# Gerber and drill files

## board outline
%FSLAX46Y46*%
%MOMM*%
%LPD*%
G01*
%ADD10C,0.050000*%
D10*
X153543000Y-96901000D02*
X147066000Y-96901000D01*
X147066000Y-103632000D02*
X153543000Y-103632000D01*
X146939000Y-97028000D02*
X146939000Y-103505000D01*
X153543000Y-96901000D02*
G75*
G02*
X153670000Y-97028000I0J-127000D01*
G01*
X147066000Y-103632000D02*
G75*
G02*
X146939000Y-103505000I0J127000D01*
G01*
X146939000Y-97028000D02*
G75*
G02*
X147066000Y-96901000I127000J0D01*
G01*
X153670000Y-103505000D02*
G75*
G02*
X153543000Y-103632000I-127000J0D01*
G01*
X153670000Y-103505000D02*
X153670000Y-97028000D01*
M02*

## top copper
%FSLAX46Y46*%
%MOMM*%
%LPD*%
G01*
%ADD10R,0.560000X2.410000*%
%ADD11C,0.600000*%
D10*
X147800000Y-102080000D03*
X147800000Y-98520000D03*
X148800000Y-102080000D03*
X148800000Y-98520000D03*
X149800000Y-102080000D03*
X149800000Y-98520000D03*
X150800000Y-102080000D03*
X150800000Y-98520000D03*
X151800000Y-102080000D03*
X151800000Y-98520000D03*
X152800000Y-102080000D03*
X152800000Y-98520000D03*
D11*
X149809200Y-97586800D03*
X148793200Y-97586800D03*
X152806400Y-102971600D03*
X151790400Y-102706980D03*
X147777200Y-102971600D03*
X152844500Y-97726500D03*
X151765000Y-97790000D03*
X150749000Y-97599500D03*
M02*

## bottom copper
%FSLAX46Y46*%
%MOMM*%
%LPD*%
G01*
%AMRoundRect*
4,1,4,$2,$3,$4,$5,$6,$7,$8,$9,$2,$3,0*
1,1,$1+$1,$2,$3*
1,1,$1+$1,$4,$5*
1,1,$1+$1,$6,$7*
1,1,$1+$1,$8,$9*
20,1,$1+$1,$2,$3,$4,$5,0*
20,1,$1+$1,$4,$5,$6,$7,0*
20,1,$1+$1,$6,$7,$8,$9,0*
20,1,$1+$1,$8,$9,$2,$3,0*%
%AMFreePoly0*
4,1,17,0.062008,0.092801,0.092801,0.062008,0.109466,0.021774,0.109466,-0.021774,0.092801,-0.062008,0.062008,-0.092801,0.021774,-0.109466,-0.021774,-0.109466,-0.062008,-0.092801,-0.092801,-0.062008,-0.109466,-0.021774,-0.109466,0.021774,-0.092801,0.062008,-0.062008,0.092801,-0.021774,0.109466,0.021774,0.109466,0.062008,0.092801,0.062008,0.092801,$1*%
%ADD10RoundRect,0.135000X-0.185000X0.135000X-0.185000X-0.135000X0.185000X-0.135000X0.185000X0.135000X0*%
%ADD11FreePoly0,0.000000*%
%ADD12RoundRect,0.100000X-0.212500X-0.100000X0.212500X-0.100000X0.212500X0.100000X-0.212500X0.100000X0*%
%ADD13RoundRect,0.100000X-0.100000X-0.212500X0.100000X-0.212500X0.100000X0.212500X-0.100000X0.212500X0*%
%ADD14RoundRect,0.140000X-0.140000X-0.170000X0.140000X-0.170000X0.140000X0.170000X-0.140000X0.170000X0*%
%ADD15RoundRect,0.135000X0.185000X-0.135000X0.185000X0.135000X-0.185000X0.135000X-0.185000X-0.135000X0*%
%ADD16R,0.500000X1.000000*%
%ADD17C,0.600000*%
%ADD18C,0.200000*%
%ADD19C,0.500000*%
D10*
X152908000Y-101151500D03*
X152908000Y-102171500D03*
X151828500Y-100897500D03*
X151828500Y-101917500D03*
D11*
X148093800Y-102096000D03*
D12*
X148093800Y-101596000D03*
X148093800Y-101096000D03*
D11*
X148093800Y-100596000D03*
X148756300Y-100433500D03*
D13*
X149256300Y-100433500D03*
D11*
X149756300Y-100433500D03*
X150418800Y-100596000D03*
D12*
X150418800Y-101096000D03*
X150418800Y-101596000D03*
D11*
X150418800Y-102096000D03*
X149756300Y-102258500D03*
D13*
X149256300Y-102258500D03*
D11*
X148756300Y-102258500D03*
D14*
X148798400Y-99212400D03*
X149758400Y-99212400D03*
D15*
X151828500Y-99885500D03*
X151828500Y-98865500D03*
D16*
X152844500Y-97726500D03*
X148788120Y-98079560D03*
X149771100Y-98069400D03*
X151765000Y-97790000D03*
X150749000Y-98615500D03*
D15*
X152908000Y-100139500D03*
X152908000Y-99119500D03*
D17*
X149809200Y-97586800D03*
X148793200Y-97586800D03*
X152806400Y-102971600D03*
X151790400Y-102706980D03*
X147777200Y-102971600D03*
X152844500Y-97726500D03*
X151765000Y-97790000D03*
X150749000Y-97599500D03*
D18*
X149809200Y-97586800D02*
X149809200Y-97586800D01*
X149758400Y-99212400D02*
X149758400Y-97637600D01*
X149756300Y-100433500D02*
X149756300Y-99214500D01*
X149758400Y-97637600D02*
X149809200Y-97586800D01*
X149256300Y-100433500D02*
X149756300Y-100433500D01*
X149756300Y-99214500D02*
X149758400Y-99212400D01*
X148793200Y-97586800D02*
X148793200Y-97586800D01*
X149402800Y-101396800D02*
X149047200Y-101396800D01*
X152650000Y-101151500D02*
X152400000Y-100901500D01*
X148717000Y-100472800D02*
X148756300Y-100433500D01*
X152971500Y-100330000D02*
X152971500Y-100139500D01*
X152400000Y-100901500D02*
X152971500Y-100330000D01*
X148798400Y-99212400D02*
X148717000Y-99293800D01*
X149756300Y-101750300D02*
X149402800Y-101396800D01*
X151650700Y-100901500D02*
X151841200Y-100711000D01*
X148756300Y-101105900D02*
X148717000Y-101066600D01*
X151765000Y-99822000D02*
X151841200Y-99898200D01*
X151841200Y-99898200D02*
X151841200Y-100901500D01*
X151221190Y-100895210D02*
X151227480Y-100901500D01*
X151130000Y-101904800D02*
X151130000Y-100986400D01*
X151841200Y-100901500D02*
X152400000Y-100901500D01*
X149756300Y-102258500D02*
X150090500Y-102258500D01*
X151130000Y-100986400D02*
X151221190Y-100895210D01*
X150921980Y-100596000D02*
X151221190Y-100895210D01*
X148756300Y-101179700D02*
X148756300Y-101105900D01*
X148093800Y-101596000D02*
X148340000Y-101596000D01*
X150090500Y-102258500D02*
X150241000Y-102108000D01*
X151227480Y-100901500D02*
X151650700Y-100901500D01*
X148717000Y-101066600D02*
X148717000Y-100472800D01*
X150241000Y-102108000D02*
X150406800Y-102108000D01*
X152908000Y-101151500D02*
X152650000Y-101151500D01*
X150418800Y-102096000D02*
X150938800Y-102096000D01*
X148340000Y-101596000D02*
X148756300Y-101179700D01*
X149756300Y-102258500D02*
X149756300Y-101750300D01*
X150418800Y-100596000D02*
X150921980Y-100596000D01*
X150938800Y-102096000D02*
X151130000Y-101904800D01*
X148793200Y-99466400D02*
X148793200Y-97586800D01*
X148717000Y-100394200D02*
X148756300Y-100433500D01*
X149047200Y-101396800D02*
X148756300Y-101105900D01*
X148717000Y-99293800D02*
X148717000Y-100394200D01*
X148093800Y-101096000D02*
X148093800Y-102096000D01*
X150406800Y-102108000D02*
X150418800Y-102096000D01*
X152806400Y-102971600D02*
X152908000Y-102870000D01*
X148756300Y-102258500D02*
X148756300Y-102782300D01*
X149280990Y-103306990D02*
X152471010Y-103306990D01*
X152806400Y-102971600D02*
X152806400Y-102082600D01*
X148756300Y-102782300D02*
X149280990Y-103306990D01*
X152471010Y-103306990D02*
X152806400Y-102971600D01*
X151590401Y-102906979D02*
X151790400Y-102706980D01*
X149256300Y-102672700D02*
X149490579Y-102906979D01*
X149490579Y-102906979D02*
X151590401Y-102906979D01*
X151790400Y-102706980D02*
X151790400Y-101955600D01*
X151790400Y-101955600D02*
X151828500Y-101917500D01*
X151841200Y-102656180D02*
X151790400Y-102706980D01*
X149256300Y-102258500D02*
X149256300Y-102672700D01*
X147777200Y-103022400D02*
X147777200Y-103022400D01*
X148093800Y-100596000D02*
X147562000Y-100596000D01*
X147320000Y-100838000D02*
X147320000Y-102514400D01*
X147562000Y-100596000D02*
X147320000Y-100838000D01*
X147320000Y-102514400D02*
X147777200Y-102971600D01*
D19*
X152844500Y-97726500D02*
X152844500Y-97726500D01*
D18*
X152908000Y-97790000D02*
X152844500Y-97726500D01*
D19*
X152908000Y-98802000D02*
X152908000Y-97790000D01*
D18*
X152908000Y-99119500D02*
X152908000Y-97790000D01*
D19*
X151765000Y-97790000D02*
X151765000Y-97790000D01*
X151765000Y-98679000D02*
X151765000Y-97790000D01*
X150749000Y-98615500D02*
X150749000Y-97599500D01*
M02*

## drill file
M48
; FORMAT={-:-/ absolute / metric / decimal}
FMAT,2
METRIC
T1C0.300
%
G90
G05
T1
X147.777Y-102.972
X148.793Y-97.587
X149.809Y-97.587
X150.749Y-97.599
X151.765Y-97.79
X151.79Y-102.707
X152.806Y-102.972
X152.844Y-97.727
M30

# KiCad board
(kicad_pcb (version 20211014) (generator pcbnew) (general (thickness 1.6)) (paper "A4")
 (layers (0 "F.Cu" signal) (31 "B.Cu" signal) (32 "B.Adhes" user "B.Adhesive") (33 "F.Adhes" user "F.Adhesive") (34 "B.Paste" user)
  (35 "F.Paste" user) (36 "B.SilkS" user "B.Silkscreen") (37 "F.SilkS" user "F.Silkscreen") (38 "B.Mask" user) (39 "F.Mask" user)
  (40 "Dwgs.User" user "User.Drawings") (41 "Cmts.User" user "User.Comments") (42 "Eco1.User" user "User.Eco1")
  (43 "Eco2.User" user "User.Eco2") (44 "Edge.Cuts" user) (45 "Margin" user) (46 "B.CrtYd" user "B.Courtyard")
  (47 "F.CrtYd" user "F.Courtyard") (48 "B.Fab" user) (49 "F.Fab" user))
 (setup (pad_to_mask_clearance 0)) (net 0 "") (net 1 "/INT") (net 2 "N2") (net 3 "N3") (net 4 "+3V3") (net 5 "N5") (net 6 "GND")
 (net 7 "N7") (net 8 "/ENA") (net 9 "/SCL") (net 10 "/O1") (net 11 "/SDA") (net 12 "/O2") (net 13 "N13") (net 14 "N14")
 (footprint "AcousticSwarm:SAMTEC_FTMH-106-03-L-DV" (layer "F.Cu") (at 150.3 100.3)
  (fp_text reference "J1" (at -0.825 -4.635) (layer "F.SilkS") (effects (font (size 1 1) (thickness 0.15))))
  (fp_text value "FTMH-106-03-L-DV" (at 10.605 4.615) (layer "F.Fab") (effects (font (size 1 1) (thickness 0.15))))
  (pad "01" smd rect locked (at -2.5 1.78) (size 0.56 2.41) (layers "F.Cu" "F.Paste" "F.Mask") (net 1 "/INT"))
  (pad "02" smd rect locked (at -2.5 -1.78) (size 0.56 2.41) (layers "F.Cu" "F.Paste" "F.Mask") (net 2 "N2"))
  (pad "03" smd rect locked (at -1.5 1.78) (size 0.56 2.41) (layers "F.Cu" "F.Paste" "F.Mask") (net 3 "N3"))
  (pad "04" smd rect locked (at -1.5 -1.78) (size 0.56 2.41) (layers "F.Cu" "F.Paste" "F.Mask") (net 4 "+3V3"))
  (pad "05" smd rect locked (at -0.5 1.78) (size 0.56 2.41) (layers "F.Cu" "F.Paste" "F.Mask") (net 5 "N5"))
  (pad "06" smd rect locked (at -0.5 -1.78) (size 0.56 2.41) (layers "F.Cu" "F.Paste" "F.Mask") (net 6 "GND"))
  (pad "07" smd rect locked (at 0.5 1.78) (size 0.56 2.41) (layers "F.Cu" "F.Paste" "F.Mask") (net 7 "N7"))
  (pad "08" smd rect locked (at 0.5 -1.78) (size 0.56 2.41) (layers "F.Cu" "F.Paste" "F.Mask") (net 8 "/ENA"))
  (pad "09" smd rect locked (at 1.5 1.78) (size 0.56 2.41) (layers "F.Cu" "F.Paste" "F.Mask") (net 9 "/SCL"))
  (pad "10" smd rect locked (at 1.5 -1.78) (size 0.56 2.41) (layers "F.Cu" "F.Paste" "F.Mask") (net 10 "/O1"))
  (pad "11" smd rect locked (at 2.5 1.78) (size 0.56 2.41) (layers "F.Cu" "F.Paste" "F.Mask") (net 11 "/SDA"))
  (pad "12" smd rect locked (at 2.5 -1.78) (size 0.56 2.41) (layers "F.Cu" "F.Paste" "F.Mask") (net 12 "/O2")))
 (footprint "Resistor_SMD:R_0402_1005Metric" (layer "B.Cu") (at 152.908 101.6615 -90)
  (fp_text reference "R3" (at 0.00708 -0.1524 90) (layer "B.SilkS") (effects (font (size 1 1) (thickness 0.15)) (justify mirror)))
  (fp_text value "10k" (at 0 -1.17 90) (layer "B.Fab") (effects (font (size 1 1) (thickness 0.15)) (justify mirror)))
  (pad "1" smd roundrect locked (at -0.51 0 270) (size 0.54 0.64) (layers "B.Cu" "B.Paste" "B.Mask") (roundrect_rratio 0.25) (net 4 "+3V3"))
  (pad "2" smd roundrect locked (at 0.51 0 270) (size 0.54 0.64) (layers "B.Cu" "B.Paste" "B.Mask") (roundrect_rratio 0.25) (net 11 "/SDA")))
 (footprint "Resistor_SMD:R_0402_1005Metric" (layer "B.Cu") (at 151.8285 101.4075 -90)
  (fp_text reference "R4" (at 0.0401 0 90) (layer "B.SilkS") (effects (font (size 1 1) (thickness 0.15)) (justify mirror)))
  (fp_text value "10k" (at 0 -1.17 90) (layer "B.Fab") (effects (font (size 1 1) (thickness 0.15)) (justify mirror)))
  (pad "1" smd roundrect locked (at -0.51 0 270) (size 0.54 0.64) (layers "B.Cu" "B.Paste" "B.Mask") (roundrect_rratio 0.25) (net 4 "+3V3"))
  (pad "2" smd roundrect locked (at 0.51 0 270) (size 0.54 0.64) (layers "B.Cu" "B.Paste" "B.Mask") (roundrect_rratio 0.25) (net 9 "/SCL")))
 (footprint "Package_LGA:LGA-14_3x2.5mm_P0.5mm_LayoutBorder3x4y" (layer "B.Cu") (at 149.2563 101.346)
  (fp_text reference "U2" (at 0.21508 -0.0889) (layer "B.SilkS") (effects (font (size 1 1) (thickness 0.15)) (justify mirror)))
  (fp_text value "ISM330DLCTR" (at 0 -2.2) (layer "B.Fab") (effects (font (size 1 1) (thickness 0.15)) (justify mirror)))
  (pad "1" smd custom locked (at -1.1625 0.75) (size 0.223223 0.223223) (layers "B.Cu" "B.Paste" "B.Mask") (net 4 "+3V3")
   (options (clearance outline) (anchor circle)) (primitives))
  (pad "2" smd roundrect locked (at -1.1625 0.25) (size 0.625 0.4) (layers "B.Cu" "B.Paste" "B.Mask") (roundrect_rratio 0.25) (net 4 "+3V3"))
  (pad "3" smd roundrect locked (at -1.1625 -0.25) (size 0.625 0.4) (layers "B.Cu" "B.Paste" "B.Mask") (roundrect_rratio 0.25)
   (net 4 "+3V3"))
  (pad "4" smd custom locked (at -1.1625 -0.75) (size 0.223223 0.223223) (layers "B.Cu" "B.Paste" "B.Mask") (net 1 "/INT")
   (options (clearance outline) (anchor circle)) (primitives))
  (pad "5" smd custom locked (at -0.5 -0.9125) (size 0.223223 0.223223) (layers "B.Cu" "B.Paste" "B.Mask") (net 4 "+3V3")
   (options (clearance outline) (anchor circle)) (primitives))
  (pad "6" smd roundrect locked (at 0 -0.9125) (size 0.4 0.625) (layers "B.Cu" "B.Paste" "B.Mask") (roundrect_rratio 0.25) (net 6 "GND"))
  (pad "7" smd custom locked (at 0.5 -0.9125) (size 0.223223 0.223223) (layers "B.Cu" "B.Paste" "B.Mask") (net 6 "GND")
   (options (clearance outline) (anchor circle)) (primitives))
  (pad "8" smd custom locked (at 1.1625 -0.75) (size 0.223223 0.223223) (layers "B.Cu" "B.Paste" "B.Mask") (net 4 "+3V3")
   (options (clearance outline) (anchor circle)) (primitives))
  (pad "9" smd roundrect locked (at 1.1625 -0.25) (size 0.625 0.4) (layers "B.Cu" "B.Paste" "B.Mask") (roundrect_rratio 0.25) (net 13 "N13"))
  (pad "10" smd roundrect locked (at 1.1625 0.25) (size 0.625 0.4) (layers "B.Cu" "B.Paste" "B.Mask") (roundrect_rratio 0.25) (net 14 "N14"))
  (pad "11" smd custom locked (at 1.1625 0.75) (size 0.223223 0.223223) (layers "B.Cu" "B.Paste" "B.Mask") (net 4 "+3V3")
   (options (clearance outline) (anchor circle)) (primitives))
  (pad "12" smd custom locked (at 0.5 0.9125) (size 0.223223 0.223223) (layers "B.Cu" "B.Paste" "B.Mask") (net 4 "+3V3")
   (options (clearance outline) (anchor circle)) (primitives))
  (pad "13" smd roundrect locked (at 0 0.9125) (size 0.4 0.625) (layers "B.Cu" "B.Paste" "B.Mask") (roundrect_rratio 0.25) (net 9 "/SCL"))
  (pad "14" smd custom locked (at -0.5 0.9125) (size 0.223223 0.223223) (layers "B.Cu" "B.Paste" "B.Mask") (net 11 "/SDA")
   (options (clearance outline) (anchor circle)) (primitives)))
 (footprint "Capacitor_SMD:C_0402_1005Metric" (layer "B.Cu") (at 149.2784 99.2124)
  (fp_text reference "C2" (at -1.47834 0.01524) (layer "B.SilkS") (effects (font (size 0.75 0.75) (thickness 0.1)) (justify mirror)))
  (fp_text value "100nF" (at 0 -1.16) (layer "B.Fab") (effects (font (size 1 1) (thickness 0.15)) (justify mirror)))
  (pad "1" smd roundrect locked (at -0.48 0) (size 0.56 0.62) (layers "B.Cu" "B.Paste" "B.Mask") (roundrect_rratio 0.25) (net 4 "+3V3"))
  (pad "2" smd roundrect locked (at 0.48 0) (size 0.56 0.62) (layers "B.Cu" "B.Paste" "B.Mask") (roundrect_rratio 0.25) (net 6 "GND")))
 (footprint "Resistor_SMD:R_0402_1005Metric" (layer "B.Cu") (at 151.8285 99.3755 90)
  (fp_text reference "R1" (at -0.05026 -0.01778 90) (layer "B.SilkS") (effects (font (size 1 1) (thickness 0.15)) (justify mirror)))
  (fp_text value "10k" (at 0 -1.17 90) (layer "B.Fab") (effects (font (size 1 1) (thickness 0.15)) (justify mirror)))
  (pad "1" smd roundrect locked (at -0.51 0 90) (size 0.54 0.64) (layers "B.Cu" "B.Paste" "B.Mask") (roundrect_rratio 0.25) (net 4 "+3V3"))
  (pad "2" smd roundrect locked (at 0.51 0 90) (size 0.54 0.64) (layers "B.Cu" "B.Paste" "B.Mask") (roundrect_rratio 0.25) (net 10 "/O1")))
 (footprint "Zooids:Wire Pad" (layer "B.Cu") (at 152.781 99.6315)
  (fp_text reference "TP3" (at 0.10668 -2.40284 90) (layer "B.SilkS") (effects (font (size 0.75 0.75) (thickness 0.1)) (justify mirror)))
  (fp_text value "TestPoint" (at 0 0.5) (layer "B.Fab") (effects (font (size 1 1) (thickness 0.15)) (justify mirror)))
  (pad "1" smd rect locked (at 0.0635 -1.905) (size 0.5 1) (layers "B.Cu" "B.Paste" "B.Mask") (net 12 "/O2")))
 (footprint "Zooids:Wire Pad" (layer "B.Cu") (at 148.72462 99.98456)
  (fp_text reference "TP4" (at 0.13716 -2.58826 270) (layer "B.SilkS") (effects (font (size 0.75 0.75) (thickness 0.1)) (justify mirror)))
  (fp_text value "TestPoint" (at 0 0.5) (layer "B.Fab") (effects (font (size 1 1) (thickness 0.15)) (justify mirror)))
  (pad "1" smd rect locked (at 0.0635 -1.905) (size 0.5 1) (layers "B.Cu" "B.Paste" "B.Mask") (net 4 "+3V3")))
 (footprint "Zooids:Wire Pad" (layer "B.Cu") (at 149.7076 99.9744)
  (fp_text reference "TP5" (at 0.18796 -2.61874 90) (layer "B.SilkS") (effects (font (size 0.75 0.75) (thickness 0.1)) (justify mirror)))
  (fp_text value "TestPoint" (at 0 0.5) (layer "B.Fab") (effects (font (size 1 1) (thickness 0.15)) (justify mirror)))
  (pad "1" smd rect locked (at 0.0635 -1.905) (size 0.5 1) (layers "B.Cu" "B.Paste" "B.Mask") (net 6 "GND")))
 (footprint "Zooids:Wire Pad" (layer "B.Cu") (at 151.7015 99.695)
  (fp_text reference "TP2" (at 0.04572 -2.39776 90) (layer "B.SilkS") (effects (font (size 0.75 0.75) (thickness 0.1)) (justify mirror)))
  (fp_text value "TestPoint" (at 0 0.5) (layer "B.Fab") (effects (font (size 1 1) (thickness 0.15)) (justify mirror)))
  (pad "1" smd rect locked (at 0.0635 -1.905) (size 0.5 1) (layers "B.Cu" "B.Paste" "B.Mask") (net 10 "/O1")))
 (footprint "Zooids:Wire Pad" (layer "B.Cu") (at 150.6855 100.5205)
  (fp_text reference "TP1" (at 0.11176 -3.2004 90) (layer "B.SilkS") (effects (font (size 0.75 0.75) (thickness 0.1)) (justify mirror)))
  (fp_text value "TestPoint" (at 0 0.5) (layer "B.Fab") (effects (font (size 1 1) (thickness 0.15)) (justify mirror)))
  (pad "1" smd rect locked (at 0.0635 -1.905) (size 0.5 1) (layers "B.Cu" "B.Paste" "B.Mask") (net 8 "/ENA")))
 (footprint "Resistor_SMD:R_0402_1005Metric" (layer "B.Cu") (at 152.908 99.6295 90)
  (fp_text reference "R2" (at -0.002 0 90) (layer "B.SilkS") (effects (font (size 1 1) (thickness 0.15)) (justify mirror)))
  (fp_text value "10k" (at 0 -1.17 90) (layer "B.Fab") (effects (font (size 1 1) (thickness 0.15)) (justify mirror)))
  (pad "1" smd roundrect locked (at -0.51 0 90) (size 0.54 0.64) (layers "B.Cu" "B.Paste" "B.Mask") (roundrect_rratio 0.25) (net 4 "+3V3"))
  (pad "2" smd roundrect locked (at 0.51 0 90) (size 0.54 0.64) (layers "B.Cu" "B.Paste" "B.Mask") (roundrect_rratio 0.25) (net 12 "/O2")))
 (gr_line (start 153.543 96.901) (end 147.066 96.901) (layer "Edge.Cuts") (width 0.05))
 (gr_line (start 147.066 103.632) (end 153.543 103.632) (layer "Edge.Cuts") (width 0.05))
 (gr_line (start 146.939 97.028) (end 146.939 103.505) (layer "Edge.Cuts") (width 0.05))
 (gr_arc (start 153.543 96.901) (mid 153.632803 96.938197) (end 153.67 97.028) (layer "Edge.Cuts") (width 0.05))
 (gr_arc (start 147.066 103.632) (mid 146.976197 103.594803) (end 146.939 103.505) (layer "Edge.Cuts") (width 0.05))
 (gr_arc (start 146.939 97.028) (mid 146.976197 96.938197) (end 147.066 96.901) (layer "Edge.Cuts") (width 0.05))
 (gr_arc (start 153.67 103.505) (mid 153.632803 103.594803) (end 153.543 103.632) (layer "Edge.Cuts") (width 0.05))
 (gr_line (start 153.67 103.505) (end 153.67 97.028) (layer "Edge.Cuts") (width 0.05))
 (via (at 149.8092 97.5868) (size 0.6) (drill 0.3) (layers "F.Cu" "B.Cu") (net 6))
 (segment (start 149.8092 97.5868) (end 149.8092 97.5868) (width 0.2) (layer "B.Cu") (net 6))
 (segment (start 149.7584 99.2124) (end 149.7584 97.6376) (width 0.2) (layer "B.Cu") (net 6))
 (segment (start 149.7563 100.4335) (end 149.7563 99.2145) (width 0.2) (layer "B.Cu") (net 6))
 (segment (start 149.7584 97.6376) (end 149.8092 97.5868) (width 0.2) (layer "B.Cu") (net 6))
 (segment (start 149.2563 100.4335) (end 149.7563 100.4335) (width 0.2) (layer "B.Cu") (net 6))
 (segment (start 149.7563 99.2145) (end 149.7584 99.2124) (width 0.2) (layer "B.Cu") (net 6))
 (via (at 148.7932 97.5868) (size 0.6) (drill 0.3) (layers "F.Cu" "B.Cu") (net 4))
 (segment (start 148.7932 97.5868) (end 148.7932 97.5868) (width 0.2) (layer "B.Cu") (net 4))
 (segment (start 149.4028 101.3968) (end 149.0472 101.3968) (width 0.2) (layer "B.Cu") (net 4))
 (segment (start 152.65 101.1515) (end 152.4 100.9015) (width 0.2) (layer "B.Cu") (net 4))
 (segment (start 148.717 100.4728) (end 148.7563 100.4335) (width 0.2) (layer "B.Cu") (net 4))
 (segment (start 152.9715 100.33) (end 152.9715 100.1395) (width 0.2) (layer "B.Cu") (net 4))
 (segment (start 152.4 100.9015) (end 152.9715 100.33) (width 0.2) (layer "B.Cu") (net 4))
 (segment (start 148.7984 99.2124) (end 148.717 99.2938) (width 0.2) (layer "B.Cu") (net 4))
 (segment (start 149.7563 101.7503) (end 149.4028 101.3968) (width 0.2) (layer "B.Cu") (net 4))
 (segment (start 151.6507 100.9015) (end 151.8412 100.711) (width 0.2) (layer "B.Cu") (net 4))
 (segment (start 148.7563 101.1059) (end 148.717 101.0666) (width 0.2) (layer "B.Cu") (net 4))
 (segment (start 151.765 99.822) (end 151.8412 99.8982) (width 0.2) (layer "B.Cu") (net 4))
 (segment (start 151.8412 99.8982) (end 151.8412 100.9015) (width 0.2) (layer "B.Cu") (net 4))
 (segment (start 151.22119 100.89521) (end 151.22748 100.9015) (width 0.2) (layer "B.Cu") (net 4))
 (segment (start 151.13 101.9048) (end 151.13 100.9864) (width 0.2) (layer "B.Cu") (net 4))
 (segment (start 151.8412 100.9015) (end 152.4 100.9015) (width 0.2) (layer "B.Cu") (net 4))
 (segment (start 149.7563 102.2585) (end 150.0905 102.2585) (width 0.2) (layer "B.Cu") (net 4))
 (segment (start 151.13 100.9864) (end 151.22119 100.89521) (width 0.2) (layer "B.Cu") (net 4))
 (segment (start 150.92198 100.596) (end 151.22119 100.89521) (width 0.2) (layer "B.Cu") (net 4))
 (segment (start 148.7563 101.1797) (end 148.7563 101.1059) (width 0.2) (layer "B.Cu") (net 4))
 (segment (start 148.0938 101.596) (end 148.34 101.596) (width 0.2) (layer "B.Cu") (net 4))
 (segment (start 150.0905 102.2585) (end 150.241 102.108) (width 0.2) (layer "B.Cu") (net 4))
 (segment (start 151.22748 100.9015) (end 151.6507 100.9015) (width 0.2) (layer "B.Cu") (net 4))
 (segment (start 148.717 101.0666) (end 148.717 100.4728) (width 0.2) (layer "B.Cu") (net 4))
 (segment (start 150.241 102.108) (end 150.4068 102.108) (width 0.2) (layer "B.Cu") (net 4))
 (segment (start 152.908 101.1515) (end 152.65 101.1515) (width 0.2) (layer "B.Cu") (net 4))
 (segment (start 150.4188 102.096) (end 150.9388 102.096) (width 0.2) (layer "B.Cu") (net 4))
 (segment (start 148.34 101.596) (end 148.7563 101.1797) (width 0.2) (layer "B.Cu") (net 4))
 (segment (start 149.7563 102.2585) (end 149.7563 101.7503) (width 0.2) (layer "B.Cu") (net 4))
 (segment (start 150.4188 100.596) (end 150.92198 100.596) (width 0.2) (layer "B.Cu") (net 4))
 (segment (start 150.9388 102.096) (end 151.13 101.9048) (width 0.2) (layer "B.Cu") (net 4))
 (segment (start 148.7932 99.4664) (end 148.7932 97.5868) (width 0.2) (layer "B.Cu") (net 4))
 (segment (start 148.717 100.3942) (end 148.7563 100.4335) (width 0.2) (layer "B.Cu") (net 4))
 (segment (start 149.0472 101.3968) (end 148.7563 101.1059) (width 0.2) (layer "B.Cu") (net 4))
 (segment (start 148.717 99.2938) (end 148.717 100.3942) (width 0.2) (layer "B.Cu") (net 4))
 (segment (start 148.0938 101.096) (end 148.0938 102.096) (width 0.2) (layer "B.Cu") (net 4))
 (segment (start 150.4068 102.108) (end 150.4188 102.096) (width 0.2) (layer "B.Cu") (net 4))
 (via (at 152.8064 102.9716) (size 0.6) (drill 0.3) (layers "F.Cu" "B.Cu") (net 11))
 (segment (start 152.8064 102.9716) (end 152.908 102.87) (width 0.2) (layer "B.Cu") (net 11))
 (segment (start 148.7563 102.2585) (end 148.7563 102.7823) (width 0.2) (layer "B.Cu") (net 11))
 (segment (start 149.28099 103.30699) (end 152.47101 103.30699) (width 0.2) (layer "B.Cu") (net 11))
 (segment (start 152.8064 102.9716) (end 152.8064 102.0826) (width 0.2) (layer "B.Cu") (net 11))
 (segment (start 148.7563 102.7823) (end 149.28099 103.30699) (width 0.2) (layer "B.Cu") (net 11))
 (segment (start 152.47101 103.30699) (end 152.8064 102.9716) (width 0.2) (layer "B.Cu") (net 11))
 (via (at 151.7904 102.70698) (size 0.6) (drill 0.3) (layers "F.Cu" "B.Cu") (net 9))
 (segment (start 151.590401 102.906979) (end 151.7904 102.70698) (width 0.2) (layer "B.Cu") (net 9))
 (segment (start 149.2563 102.6727) (end 149.490579 102.906979) (width 0.2) (layer "B.Cu") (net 9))
 (segment (start 149.490579 102.906979) (end 151.590401 102.906979) (width 0.2) (layer "B.Cu") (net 9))
 (segment (start 151.7904 102.70698) (end 151.7904 101.9556) (width 0.2) (layer "B.Cu") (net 9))
 (segment (start 151.7904 101.9556) (end 151.8285 101.9175) (width 0.2) (layer "B.Cu") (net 9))
 (segment (start 151.8412 102.65618) (end 151.7904 102.70698) (width 0.2) (layer "B.Cu") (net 9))
 (segment (start 149.2563 102.2585) (end 149.2563 102.6727) (width 0.2) (layer "B.Cu") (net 9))
 (via (at 147.7772 102.9716) (size 0.6) (drill 0.3) (layers "F.Cu" "B.Cu") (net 1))
 (segment (start 147.7772 103.0224) (end 147.7772 103.0224) (width 0.2) (layer "B.Cu") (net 1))
 (segment (start 148.0938 100.596) (end 147.562 100.596) (width 0.2) (layer "B.Cu") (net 1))
 (segment (start 147.32 100.838) (end 147.32 102.5144) (width 0.2) (layer "B.Cu") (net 1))
 (segment (start 147.562 100.596) (end 147.32 100.838) (width 0.2) (layer "B.Cu") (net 1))
 (segment (start 147.32 102.5144) (end 147.7772 102.9716) (width 0.2) (layer "B.Cu") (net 1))
 (via (at 152.8445 97.7265) (size 0.6) (drill 0.3) (layers "F.Cu" "B.Cu") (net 12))
 (segment (start 152.8445 97.7265) (end 152.8445 97.7265) (width 0.5) (layer "B.Cu") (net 12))
 (segment (start 152.908 97.79) (end 152.8445 97.7265) (width 0.2) (layer "B.Cu") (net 12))
 (segment (start 152.908 98.802) (end 152.908 97.79) (width 0.5) (layer "B.Cu") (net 12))
 (segment (start 152.908 99.1195) (end 152.908 97.79) (width 0.2) (layer "B.Cu") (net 12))
 (via (at 151.765 97.79) (size 0.6) (drill 0.3) (layers "F.Cu" "B.Cu") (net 10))
 (segment (start 151.765 97.79) (end 151.765 97.79) (width 0.5) (layer "B.Cu") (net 10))
 (segment (start 151.765 98.679) (end 151.765 97.79) (width 0.5) (layer "B.Cu") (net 10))
 (via (at 150.749 97.5995) (size 0.6) (drill 0.3) (layers "F.Cu" "B.Cu") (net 8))
 (segment (start 150.749 98.6155) (end 150.749 97.5995) (width 0.5) (layer "B.Cu") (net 8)))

